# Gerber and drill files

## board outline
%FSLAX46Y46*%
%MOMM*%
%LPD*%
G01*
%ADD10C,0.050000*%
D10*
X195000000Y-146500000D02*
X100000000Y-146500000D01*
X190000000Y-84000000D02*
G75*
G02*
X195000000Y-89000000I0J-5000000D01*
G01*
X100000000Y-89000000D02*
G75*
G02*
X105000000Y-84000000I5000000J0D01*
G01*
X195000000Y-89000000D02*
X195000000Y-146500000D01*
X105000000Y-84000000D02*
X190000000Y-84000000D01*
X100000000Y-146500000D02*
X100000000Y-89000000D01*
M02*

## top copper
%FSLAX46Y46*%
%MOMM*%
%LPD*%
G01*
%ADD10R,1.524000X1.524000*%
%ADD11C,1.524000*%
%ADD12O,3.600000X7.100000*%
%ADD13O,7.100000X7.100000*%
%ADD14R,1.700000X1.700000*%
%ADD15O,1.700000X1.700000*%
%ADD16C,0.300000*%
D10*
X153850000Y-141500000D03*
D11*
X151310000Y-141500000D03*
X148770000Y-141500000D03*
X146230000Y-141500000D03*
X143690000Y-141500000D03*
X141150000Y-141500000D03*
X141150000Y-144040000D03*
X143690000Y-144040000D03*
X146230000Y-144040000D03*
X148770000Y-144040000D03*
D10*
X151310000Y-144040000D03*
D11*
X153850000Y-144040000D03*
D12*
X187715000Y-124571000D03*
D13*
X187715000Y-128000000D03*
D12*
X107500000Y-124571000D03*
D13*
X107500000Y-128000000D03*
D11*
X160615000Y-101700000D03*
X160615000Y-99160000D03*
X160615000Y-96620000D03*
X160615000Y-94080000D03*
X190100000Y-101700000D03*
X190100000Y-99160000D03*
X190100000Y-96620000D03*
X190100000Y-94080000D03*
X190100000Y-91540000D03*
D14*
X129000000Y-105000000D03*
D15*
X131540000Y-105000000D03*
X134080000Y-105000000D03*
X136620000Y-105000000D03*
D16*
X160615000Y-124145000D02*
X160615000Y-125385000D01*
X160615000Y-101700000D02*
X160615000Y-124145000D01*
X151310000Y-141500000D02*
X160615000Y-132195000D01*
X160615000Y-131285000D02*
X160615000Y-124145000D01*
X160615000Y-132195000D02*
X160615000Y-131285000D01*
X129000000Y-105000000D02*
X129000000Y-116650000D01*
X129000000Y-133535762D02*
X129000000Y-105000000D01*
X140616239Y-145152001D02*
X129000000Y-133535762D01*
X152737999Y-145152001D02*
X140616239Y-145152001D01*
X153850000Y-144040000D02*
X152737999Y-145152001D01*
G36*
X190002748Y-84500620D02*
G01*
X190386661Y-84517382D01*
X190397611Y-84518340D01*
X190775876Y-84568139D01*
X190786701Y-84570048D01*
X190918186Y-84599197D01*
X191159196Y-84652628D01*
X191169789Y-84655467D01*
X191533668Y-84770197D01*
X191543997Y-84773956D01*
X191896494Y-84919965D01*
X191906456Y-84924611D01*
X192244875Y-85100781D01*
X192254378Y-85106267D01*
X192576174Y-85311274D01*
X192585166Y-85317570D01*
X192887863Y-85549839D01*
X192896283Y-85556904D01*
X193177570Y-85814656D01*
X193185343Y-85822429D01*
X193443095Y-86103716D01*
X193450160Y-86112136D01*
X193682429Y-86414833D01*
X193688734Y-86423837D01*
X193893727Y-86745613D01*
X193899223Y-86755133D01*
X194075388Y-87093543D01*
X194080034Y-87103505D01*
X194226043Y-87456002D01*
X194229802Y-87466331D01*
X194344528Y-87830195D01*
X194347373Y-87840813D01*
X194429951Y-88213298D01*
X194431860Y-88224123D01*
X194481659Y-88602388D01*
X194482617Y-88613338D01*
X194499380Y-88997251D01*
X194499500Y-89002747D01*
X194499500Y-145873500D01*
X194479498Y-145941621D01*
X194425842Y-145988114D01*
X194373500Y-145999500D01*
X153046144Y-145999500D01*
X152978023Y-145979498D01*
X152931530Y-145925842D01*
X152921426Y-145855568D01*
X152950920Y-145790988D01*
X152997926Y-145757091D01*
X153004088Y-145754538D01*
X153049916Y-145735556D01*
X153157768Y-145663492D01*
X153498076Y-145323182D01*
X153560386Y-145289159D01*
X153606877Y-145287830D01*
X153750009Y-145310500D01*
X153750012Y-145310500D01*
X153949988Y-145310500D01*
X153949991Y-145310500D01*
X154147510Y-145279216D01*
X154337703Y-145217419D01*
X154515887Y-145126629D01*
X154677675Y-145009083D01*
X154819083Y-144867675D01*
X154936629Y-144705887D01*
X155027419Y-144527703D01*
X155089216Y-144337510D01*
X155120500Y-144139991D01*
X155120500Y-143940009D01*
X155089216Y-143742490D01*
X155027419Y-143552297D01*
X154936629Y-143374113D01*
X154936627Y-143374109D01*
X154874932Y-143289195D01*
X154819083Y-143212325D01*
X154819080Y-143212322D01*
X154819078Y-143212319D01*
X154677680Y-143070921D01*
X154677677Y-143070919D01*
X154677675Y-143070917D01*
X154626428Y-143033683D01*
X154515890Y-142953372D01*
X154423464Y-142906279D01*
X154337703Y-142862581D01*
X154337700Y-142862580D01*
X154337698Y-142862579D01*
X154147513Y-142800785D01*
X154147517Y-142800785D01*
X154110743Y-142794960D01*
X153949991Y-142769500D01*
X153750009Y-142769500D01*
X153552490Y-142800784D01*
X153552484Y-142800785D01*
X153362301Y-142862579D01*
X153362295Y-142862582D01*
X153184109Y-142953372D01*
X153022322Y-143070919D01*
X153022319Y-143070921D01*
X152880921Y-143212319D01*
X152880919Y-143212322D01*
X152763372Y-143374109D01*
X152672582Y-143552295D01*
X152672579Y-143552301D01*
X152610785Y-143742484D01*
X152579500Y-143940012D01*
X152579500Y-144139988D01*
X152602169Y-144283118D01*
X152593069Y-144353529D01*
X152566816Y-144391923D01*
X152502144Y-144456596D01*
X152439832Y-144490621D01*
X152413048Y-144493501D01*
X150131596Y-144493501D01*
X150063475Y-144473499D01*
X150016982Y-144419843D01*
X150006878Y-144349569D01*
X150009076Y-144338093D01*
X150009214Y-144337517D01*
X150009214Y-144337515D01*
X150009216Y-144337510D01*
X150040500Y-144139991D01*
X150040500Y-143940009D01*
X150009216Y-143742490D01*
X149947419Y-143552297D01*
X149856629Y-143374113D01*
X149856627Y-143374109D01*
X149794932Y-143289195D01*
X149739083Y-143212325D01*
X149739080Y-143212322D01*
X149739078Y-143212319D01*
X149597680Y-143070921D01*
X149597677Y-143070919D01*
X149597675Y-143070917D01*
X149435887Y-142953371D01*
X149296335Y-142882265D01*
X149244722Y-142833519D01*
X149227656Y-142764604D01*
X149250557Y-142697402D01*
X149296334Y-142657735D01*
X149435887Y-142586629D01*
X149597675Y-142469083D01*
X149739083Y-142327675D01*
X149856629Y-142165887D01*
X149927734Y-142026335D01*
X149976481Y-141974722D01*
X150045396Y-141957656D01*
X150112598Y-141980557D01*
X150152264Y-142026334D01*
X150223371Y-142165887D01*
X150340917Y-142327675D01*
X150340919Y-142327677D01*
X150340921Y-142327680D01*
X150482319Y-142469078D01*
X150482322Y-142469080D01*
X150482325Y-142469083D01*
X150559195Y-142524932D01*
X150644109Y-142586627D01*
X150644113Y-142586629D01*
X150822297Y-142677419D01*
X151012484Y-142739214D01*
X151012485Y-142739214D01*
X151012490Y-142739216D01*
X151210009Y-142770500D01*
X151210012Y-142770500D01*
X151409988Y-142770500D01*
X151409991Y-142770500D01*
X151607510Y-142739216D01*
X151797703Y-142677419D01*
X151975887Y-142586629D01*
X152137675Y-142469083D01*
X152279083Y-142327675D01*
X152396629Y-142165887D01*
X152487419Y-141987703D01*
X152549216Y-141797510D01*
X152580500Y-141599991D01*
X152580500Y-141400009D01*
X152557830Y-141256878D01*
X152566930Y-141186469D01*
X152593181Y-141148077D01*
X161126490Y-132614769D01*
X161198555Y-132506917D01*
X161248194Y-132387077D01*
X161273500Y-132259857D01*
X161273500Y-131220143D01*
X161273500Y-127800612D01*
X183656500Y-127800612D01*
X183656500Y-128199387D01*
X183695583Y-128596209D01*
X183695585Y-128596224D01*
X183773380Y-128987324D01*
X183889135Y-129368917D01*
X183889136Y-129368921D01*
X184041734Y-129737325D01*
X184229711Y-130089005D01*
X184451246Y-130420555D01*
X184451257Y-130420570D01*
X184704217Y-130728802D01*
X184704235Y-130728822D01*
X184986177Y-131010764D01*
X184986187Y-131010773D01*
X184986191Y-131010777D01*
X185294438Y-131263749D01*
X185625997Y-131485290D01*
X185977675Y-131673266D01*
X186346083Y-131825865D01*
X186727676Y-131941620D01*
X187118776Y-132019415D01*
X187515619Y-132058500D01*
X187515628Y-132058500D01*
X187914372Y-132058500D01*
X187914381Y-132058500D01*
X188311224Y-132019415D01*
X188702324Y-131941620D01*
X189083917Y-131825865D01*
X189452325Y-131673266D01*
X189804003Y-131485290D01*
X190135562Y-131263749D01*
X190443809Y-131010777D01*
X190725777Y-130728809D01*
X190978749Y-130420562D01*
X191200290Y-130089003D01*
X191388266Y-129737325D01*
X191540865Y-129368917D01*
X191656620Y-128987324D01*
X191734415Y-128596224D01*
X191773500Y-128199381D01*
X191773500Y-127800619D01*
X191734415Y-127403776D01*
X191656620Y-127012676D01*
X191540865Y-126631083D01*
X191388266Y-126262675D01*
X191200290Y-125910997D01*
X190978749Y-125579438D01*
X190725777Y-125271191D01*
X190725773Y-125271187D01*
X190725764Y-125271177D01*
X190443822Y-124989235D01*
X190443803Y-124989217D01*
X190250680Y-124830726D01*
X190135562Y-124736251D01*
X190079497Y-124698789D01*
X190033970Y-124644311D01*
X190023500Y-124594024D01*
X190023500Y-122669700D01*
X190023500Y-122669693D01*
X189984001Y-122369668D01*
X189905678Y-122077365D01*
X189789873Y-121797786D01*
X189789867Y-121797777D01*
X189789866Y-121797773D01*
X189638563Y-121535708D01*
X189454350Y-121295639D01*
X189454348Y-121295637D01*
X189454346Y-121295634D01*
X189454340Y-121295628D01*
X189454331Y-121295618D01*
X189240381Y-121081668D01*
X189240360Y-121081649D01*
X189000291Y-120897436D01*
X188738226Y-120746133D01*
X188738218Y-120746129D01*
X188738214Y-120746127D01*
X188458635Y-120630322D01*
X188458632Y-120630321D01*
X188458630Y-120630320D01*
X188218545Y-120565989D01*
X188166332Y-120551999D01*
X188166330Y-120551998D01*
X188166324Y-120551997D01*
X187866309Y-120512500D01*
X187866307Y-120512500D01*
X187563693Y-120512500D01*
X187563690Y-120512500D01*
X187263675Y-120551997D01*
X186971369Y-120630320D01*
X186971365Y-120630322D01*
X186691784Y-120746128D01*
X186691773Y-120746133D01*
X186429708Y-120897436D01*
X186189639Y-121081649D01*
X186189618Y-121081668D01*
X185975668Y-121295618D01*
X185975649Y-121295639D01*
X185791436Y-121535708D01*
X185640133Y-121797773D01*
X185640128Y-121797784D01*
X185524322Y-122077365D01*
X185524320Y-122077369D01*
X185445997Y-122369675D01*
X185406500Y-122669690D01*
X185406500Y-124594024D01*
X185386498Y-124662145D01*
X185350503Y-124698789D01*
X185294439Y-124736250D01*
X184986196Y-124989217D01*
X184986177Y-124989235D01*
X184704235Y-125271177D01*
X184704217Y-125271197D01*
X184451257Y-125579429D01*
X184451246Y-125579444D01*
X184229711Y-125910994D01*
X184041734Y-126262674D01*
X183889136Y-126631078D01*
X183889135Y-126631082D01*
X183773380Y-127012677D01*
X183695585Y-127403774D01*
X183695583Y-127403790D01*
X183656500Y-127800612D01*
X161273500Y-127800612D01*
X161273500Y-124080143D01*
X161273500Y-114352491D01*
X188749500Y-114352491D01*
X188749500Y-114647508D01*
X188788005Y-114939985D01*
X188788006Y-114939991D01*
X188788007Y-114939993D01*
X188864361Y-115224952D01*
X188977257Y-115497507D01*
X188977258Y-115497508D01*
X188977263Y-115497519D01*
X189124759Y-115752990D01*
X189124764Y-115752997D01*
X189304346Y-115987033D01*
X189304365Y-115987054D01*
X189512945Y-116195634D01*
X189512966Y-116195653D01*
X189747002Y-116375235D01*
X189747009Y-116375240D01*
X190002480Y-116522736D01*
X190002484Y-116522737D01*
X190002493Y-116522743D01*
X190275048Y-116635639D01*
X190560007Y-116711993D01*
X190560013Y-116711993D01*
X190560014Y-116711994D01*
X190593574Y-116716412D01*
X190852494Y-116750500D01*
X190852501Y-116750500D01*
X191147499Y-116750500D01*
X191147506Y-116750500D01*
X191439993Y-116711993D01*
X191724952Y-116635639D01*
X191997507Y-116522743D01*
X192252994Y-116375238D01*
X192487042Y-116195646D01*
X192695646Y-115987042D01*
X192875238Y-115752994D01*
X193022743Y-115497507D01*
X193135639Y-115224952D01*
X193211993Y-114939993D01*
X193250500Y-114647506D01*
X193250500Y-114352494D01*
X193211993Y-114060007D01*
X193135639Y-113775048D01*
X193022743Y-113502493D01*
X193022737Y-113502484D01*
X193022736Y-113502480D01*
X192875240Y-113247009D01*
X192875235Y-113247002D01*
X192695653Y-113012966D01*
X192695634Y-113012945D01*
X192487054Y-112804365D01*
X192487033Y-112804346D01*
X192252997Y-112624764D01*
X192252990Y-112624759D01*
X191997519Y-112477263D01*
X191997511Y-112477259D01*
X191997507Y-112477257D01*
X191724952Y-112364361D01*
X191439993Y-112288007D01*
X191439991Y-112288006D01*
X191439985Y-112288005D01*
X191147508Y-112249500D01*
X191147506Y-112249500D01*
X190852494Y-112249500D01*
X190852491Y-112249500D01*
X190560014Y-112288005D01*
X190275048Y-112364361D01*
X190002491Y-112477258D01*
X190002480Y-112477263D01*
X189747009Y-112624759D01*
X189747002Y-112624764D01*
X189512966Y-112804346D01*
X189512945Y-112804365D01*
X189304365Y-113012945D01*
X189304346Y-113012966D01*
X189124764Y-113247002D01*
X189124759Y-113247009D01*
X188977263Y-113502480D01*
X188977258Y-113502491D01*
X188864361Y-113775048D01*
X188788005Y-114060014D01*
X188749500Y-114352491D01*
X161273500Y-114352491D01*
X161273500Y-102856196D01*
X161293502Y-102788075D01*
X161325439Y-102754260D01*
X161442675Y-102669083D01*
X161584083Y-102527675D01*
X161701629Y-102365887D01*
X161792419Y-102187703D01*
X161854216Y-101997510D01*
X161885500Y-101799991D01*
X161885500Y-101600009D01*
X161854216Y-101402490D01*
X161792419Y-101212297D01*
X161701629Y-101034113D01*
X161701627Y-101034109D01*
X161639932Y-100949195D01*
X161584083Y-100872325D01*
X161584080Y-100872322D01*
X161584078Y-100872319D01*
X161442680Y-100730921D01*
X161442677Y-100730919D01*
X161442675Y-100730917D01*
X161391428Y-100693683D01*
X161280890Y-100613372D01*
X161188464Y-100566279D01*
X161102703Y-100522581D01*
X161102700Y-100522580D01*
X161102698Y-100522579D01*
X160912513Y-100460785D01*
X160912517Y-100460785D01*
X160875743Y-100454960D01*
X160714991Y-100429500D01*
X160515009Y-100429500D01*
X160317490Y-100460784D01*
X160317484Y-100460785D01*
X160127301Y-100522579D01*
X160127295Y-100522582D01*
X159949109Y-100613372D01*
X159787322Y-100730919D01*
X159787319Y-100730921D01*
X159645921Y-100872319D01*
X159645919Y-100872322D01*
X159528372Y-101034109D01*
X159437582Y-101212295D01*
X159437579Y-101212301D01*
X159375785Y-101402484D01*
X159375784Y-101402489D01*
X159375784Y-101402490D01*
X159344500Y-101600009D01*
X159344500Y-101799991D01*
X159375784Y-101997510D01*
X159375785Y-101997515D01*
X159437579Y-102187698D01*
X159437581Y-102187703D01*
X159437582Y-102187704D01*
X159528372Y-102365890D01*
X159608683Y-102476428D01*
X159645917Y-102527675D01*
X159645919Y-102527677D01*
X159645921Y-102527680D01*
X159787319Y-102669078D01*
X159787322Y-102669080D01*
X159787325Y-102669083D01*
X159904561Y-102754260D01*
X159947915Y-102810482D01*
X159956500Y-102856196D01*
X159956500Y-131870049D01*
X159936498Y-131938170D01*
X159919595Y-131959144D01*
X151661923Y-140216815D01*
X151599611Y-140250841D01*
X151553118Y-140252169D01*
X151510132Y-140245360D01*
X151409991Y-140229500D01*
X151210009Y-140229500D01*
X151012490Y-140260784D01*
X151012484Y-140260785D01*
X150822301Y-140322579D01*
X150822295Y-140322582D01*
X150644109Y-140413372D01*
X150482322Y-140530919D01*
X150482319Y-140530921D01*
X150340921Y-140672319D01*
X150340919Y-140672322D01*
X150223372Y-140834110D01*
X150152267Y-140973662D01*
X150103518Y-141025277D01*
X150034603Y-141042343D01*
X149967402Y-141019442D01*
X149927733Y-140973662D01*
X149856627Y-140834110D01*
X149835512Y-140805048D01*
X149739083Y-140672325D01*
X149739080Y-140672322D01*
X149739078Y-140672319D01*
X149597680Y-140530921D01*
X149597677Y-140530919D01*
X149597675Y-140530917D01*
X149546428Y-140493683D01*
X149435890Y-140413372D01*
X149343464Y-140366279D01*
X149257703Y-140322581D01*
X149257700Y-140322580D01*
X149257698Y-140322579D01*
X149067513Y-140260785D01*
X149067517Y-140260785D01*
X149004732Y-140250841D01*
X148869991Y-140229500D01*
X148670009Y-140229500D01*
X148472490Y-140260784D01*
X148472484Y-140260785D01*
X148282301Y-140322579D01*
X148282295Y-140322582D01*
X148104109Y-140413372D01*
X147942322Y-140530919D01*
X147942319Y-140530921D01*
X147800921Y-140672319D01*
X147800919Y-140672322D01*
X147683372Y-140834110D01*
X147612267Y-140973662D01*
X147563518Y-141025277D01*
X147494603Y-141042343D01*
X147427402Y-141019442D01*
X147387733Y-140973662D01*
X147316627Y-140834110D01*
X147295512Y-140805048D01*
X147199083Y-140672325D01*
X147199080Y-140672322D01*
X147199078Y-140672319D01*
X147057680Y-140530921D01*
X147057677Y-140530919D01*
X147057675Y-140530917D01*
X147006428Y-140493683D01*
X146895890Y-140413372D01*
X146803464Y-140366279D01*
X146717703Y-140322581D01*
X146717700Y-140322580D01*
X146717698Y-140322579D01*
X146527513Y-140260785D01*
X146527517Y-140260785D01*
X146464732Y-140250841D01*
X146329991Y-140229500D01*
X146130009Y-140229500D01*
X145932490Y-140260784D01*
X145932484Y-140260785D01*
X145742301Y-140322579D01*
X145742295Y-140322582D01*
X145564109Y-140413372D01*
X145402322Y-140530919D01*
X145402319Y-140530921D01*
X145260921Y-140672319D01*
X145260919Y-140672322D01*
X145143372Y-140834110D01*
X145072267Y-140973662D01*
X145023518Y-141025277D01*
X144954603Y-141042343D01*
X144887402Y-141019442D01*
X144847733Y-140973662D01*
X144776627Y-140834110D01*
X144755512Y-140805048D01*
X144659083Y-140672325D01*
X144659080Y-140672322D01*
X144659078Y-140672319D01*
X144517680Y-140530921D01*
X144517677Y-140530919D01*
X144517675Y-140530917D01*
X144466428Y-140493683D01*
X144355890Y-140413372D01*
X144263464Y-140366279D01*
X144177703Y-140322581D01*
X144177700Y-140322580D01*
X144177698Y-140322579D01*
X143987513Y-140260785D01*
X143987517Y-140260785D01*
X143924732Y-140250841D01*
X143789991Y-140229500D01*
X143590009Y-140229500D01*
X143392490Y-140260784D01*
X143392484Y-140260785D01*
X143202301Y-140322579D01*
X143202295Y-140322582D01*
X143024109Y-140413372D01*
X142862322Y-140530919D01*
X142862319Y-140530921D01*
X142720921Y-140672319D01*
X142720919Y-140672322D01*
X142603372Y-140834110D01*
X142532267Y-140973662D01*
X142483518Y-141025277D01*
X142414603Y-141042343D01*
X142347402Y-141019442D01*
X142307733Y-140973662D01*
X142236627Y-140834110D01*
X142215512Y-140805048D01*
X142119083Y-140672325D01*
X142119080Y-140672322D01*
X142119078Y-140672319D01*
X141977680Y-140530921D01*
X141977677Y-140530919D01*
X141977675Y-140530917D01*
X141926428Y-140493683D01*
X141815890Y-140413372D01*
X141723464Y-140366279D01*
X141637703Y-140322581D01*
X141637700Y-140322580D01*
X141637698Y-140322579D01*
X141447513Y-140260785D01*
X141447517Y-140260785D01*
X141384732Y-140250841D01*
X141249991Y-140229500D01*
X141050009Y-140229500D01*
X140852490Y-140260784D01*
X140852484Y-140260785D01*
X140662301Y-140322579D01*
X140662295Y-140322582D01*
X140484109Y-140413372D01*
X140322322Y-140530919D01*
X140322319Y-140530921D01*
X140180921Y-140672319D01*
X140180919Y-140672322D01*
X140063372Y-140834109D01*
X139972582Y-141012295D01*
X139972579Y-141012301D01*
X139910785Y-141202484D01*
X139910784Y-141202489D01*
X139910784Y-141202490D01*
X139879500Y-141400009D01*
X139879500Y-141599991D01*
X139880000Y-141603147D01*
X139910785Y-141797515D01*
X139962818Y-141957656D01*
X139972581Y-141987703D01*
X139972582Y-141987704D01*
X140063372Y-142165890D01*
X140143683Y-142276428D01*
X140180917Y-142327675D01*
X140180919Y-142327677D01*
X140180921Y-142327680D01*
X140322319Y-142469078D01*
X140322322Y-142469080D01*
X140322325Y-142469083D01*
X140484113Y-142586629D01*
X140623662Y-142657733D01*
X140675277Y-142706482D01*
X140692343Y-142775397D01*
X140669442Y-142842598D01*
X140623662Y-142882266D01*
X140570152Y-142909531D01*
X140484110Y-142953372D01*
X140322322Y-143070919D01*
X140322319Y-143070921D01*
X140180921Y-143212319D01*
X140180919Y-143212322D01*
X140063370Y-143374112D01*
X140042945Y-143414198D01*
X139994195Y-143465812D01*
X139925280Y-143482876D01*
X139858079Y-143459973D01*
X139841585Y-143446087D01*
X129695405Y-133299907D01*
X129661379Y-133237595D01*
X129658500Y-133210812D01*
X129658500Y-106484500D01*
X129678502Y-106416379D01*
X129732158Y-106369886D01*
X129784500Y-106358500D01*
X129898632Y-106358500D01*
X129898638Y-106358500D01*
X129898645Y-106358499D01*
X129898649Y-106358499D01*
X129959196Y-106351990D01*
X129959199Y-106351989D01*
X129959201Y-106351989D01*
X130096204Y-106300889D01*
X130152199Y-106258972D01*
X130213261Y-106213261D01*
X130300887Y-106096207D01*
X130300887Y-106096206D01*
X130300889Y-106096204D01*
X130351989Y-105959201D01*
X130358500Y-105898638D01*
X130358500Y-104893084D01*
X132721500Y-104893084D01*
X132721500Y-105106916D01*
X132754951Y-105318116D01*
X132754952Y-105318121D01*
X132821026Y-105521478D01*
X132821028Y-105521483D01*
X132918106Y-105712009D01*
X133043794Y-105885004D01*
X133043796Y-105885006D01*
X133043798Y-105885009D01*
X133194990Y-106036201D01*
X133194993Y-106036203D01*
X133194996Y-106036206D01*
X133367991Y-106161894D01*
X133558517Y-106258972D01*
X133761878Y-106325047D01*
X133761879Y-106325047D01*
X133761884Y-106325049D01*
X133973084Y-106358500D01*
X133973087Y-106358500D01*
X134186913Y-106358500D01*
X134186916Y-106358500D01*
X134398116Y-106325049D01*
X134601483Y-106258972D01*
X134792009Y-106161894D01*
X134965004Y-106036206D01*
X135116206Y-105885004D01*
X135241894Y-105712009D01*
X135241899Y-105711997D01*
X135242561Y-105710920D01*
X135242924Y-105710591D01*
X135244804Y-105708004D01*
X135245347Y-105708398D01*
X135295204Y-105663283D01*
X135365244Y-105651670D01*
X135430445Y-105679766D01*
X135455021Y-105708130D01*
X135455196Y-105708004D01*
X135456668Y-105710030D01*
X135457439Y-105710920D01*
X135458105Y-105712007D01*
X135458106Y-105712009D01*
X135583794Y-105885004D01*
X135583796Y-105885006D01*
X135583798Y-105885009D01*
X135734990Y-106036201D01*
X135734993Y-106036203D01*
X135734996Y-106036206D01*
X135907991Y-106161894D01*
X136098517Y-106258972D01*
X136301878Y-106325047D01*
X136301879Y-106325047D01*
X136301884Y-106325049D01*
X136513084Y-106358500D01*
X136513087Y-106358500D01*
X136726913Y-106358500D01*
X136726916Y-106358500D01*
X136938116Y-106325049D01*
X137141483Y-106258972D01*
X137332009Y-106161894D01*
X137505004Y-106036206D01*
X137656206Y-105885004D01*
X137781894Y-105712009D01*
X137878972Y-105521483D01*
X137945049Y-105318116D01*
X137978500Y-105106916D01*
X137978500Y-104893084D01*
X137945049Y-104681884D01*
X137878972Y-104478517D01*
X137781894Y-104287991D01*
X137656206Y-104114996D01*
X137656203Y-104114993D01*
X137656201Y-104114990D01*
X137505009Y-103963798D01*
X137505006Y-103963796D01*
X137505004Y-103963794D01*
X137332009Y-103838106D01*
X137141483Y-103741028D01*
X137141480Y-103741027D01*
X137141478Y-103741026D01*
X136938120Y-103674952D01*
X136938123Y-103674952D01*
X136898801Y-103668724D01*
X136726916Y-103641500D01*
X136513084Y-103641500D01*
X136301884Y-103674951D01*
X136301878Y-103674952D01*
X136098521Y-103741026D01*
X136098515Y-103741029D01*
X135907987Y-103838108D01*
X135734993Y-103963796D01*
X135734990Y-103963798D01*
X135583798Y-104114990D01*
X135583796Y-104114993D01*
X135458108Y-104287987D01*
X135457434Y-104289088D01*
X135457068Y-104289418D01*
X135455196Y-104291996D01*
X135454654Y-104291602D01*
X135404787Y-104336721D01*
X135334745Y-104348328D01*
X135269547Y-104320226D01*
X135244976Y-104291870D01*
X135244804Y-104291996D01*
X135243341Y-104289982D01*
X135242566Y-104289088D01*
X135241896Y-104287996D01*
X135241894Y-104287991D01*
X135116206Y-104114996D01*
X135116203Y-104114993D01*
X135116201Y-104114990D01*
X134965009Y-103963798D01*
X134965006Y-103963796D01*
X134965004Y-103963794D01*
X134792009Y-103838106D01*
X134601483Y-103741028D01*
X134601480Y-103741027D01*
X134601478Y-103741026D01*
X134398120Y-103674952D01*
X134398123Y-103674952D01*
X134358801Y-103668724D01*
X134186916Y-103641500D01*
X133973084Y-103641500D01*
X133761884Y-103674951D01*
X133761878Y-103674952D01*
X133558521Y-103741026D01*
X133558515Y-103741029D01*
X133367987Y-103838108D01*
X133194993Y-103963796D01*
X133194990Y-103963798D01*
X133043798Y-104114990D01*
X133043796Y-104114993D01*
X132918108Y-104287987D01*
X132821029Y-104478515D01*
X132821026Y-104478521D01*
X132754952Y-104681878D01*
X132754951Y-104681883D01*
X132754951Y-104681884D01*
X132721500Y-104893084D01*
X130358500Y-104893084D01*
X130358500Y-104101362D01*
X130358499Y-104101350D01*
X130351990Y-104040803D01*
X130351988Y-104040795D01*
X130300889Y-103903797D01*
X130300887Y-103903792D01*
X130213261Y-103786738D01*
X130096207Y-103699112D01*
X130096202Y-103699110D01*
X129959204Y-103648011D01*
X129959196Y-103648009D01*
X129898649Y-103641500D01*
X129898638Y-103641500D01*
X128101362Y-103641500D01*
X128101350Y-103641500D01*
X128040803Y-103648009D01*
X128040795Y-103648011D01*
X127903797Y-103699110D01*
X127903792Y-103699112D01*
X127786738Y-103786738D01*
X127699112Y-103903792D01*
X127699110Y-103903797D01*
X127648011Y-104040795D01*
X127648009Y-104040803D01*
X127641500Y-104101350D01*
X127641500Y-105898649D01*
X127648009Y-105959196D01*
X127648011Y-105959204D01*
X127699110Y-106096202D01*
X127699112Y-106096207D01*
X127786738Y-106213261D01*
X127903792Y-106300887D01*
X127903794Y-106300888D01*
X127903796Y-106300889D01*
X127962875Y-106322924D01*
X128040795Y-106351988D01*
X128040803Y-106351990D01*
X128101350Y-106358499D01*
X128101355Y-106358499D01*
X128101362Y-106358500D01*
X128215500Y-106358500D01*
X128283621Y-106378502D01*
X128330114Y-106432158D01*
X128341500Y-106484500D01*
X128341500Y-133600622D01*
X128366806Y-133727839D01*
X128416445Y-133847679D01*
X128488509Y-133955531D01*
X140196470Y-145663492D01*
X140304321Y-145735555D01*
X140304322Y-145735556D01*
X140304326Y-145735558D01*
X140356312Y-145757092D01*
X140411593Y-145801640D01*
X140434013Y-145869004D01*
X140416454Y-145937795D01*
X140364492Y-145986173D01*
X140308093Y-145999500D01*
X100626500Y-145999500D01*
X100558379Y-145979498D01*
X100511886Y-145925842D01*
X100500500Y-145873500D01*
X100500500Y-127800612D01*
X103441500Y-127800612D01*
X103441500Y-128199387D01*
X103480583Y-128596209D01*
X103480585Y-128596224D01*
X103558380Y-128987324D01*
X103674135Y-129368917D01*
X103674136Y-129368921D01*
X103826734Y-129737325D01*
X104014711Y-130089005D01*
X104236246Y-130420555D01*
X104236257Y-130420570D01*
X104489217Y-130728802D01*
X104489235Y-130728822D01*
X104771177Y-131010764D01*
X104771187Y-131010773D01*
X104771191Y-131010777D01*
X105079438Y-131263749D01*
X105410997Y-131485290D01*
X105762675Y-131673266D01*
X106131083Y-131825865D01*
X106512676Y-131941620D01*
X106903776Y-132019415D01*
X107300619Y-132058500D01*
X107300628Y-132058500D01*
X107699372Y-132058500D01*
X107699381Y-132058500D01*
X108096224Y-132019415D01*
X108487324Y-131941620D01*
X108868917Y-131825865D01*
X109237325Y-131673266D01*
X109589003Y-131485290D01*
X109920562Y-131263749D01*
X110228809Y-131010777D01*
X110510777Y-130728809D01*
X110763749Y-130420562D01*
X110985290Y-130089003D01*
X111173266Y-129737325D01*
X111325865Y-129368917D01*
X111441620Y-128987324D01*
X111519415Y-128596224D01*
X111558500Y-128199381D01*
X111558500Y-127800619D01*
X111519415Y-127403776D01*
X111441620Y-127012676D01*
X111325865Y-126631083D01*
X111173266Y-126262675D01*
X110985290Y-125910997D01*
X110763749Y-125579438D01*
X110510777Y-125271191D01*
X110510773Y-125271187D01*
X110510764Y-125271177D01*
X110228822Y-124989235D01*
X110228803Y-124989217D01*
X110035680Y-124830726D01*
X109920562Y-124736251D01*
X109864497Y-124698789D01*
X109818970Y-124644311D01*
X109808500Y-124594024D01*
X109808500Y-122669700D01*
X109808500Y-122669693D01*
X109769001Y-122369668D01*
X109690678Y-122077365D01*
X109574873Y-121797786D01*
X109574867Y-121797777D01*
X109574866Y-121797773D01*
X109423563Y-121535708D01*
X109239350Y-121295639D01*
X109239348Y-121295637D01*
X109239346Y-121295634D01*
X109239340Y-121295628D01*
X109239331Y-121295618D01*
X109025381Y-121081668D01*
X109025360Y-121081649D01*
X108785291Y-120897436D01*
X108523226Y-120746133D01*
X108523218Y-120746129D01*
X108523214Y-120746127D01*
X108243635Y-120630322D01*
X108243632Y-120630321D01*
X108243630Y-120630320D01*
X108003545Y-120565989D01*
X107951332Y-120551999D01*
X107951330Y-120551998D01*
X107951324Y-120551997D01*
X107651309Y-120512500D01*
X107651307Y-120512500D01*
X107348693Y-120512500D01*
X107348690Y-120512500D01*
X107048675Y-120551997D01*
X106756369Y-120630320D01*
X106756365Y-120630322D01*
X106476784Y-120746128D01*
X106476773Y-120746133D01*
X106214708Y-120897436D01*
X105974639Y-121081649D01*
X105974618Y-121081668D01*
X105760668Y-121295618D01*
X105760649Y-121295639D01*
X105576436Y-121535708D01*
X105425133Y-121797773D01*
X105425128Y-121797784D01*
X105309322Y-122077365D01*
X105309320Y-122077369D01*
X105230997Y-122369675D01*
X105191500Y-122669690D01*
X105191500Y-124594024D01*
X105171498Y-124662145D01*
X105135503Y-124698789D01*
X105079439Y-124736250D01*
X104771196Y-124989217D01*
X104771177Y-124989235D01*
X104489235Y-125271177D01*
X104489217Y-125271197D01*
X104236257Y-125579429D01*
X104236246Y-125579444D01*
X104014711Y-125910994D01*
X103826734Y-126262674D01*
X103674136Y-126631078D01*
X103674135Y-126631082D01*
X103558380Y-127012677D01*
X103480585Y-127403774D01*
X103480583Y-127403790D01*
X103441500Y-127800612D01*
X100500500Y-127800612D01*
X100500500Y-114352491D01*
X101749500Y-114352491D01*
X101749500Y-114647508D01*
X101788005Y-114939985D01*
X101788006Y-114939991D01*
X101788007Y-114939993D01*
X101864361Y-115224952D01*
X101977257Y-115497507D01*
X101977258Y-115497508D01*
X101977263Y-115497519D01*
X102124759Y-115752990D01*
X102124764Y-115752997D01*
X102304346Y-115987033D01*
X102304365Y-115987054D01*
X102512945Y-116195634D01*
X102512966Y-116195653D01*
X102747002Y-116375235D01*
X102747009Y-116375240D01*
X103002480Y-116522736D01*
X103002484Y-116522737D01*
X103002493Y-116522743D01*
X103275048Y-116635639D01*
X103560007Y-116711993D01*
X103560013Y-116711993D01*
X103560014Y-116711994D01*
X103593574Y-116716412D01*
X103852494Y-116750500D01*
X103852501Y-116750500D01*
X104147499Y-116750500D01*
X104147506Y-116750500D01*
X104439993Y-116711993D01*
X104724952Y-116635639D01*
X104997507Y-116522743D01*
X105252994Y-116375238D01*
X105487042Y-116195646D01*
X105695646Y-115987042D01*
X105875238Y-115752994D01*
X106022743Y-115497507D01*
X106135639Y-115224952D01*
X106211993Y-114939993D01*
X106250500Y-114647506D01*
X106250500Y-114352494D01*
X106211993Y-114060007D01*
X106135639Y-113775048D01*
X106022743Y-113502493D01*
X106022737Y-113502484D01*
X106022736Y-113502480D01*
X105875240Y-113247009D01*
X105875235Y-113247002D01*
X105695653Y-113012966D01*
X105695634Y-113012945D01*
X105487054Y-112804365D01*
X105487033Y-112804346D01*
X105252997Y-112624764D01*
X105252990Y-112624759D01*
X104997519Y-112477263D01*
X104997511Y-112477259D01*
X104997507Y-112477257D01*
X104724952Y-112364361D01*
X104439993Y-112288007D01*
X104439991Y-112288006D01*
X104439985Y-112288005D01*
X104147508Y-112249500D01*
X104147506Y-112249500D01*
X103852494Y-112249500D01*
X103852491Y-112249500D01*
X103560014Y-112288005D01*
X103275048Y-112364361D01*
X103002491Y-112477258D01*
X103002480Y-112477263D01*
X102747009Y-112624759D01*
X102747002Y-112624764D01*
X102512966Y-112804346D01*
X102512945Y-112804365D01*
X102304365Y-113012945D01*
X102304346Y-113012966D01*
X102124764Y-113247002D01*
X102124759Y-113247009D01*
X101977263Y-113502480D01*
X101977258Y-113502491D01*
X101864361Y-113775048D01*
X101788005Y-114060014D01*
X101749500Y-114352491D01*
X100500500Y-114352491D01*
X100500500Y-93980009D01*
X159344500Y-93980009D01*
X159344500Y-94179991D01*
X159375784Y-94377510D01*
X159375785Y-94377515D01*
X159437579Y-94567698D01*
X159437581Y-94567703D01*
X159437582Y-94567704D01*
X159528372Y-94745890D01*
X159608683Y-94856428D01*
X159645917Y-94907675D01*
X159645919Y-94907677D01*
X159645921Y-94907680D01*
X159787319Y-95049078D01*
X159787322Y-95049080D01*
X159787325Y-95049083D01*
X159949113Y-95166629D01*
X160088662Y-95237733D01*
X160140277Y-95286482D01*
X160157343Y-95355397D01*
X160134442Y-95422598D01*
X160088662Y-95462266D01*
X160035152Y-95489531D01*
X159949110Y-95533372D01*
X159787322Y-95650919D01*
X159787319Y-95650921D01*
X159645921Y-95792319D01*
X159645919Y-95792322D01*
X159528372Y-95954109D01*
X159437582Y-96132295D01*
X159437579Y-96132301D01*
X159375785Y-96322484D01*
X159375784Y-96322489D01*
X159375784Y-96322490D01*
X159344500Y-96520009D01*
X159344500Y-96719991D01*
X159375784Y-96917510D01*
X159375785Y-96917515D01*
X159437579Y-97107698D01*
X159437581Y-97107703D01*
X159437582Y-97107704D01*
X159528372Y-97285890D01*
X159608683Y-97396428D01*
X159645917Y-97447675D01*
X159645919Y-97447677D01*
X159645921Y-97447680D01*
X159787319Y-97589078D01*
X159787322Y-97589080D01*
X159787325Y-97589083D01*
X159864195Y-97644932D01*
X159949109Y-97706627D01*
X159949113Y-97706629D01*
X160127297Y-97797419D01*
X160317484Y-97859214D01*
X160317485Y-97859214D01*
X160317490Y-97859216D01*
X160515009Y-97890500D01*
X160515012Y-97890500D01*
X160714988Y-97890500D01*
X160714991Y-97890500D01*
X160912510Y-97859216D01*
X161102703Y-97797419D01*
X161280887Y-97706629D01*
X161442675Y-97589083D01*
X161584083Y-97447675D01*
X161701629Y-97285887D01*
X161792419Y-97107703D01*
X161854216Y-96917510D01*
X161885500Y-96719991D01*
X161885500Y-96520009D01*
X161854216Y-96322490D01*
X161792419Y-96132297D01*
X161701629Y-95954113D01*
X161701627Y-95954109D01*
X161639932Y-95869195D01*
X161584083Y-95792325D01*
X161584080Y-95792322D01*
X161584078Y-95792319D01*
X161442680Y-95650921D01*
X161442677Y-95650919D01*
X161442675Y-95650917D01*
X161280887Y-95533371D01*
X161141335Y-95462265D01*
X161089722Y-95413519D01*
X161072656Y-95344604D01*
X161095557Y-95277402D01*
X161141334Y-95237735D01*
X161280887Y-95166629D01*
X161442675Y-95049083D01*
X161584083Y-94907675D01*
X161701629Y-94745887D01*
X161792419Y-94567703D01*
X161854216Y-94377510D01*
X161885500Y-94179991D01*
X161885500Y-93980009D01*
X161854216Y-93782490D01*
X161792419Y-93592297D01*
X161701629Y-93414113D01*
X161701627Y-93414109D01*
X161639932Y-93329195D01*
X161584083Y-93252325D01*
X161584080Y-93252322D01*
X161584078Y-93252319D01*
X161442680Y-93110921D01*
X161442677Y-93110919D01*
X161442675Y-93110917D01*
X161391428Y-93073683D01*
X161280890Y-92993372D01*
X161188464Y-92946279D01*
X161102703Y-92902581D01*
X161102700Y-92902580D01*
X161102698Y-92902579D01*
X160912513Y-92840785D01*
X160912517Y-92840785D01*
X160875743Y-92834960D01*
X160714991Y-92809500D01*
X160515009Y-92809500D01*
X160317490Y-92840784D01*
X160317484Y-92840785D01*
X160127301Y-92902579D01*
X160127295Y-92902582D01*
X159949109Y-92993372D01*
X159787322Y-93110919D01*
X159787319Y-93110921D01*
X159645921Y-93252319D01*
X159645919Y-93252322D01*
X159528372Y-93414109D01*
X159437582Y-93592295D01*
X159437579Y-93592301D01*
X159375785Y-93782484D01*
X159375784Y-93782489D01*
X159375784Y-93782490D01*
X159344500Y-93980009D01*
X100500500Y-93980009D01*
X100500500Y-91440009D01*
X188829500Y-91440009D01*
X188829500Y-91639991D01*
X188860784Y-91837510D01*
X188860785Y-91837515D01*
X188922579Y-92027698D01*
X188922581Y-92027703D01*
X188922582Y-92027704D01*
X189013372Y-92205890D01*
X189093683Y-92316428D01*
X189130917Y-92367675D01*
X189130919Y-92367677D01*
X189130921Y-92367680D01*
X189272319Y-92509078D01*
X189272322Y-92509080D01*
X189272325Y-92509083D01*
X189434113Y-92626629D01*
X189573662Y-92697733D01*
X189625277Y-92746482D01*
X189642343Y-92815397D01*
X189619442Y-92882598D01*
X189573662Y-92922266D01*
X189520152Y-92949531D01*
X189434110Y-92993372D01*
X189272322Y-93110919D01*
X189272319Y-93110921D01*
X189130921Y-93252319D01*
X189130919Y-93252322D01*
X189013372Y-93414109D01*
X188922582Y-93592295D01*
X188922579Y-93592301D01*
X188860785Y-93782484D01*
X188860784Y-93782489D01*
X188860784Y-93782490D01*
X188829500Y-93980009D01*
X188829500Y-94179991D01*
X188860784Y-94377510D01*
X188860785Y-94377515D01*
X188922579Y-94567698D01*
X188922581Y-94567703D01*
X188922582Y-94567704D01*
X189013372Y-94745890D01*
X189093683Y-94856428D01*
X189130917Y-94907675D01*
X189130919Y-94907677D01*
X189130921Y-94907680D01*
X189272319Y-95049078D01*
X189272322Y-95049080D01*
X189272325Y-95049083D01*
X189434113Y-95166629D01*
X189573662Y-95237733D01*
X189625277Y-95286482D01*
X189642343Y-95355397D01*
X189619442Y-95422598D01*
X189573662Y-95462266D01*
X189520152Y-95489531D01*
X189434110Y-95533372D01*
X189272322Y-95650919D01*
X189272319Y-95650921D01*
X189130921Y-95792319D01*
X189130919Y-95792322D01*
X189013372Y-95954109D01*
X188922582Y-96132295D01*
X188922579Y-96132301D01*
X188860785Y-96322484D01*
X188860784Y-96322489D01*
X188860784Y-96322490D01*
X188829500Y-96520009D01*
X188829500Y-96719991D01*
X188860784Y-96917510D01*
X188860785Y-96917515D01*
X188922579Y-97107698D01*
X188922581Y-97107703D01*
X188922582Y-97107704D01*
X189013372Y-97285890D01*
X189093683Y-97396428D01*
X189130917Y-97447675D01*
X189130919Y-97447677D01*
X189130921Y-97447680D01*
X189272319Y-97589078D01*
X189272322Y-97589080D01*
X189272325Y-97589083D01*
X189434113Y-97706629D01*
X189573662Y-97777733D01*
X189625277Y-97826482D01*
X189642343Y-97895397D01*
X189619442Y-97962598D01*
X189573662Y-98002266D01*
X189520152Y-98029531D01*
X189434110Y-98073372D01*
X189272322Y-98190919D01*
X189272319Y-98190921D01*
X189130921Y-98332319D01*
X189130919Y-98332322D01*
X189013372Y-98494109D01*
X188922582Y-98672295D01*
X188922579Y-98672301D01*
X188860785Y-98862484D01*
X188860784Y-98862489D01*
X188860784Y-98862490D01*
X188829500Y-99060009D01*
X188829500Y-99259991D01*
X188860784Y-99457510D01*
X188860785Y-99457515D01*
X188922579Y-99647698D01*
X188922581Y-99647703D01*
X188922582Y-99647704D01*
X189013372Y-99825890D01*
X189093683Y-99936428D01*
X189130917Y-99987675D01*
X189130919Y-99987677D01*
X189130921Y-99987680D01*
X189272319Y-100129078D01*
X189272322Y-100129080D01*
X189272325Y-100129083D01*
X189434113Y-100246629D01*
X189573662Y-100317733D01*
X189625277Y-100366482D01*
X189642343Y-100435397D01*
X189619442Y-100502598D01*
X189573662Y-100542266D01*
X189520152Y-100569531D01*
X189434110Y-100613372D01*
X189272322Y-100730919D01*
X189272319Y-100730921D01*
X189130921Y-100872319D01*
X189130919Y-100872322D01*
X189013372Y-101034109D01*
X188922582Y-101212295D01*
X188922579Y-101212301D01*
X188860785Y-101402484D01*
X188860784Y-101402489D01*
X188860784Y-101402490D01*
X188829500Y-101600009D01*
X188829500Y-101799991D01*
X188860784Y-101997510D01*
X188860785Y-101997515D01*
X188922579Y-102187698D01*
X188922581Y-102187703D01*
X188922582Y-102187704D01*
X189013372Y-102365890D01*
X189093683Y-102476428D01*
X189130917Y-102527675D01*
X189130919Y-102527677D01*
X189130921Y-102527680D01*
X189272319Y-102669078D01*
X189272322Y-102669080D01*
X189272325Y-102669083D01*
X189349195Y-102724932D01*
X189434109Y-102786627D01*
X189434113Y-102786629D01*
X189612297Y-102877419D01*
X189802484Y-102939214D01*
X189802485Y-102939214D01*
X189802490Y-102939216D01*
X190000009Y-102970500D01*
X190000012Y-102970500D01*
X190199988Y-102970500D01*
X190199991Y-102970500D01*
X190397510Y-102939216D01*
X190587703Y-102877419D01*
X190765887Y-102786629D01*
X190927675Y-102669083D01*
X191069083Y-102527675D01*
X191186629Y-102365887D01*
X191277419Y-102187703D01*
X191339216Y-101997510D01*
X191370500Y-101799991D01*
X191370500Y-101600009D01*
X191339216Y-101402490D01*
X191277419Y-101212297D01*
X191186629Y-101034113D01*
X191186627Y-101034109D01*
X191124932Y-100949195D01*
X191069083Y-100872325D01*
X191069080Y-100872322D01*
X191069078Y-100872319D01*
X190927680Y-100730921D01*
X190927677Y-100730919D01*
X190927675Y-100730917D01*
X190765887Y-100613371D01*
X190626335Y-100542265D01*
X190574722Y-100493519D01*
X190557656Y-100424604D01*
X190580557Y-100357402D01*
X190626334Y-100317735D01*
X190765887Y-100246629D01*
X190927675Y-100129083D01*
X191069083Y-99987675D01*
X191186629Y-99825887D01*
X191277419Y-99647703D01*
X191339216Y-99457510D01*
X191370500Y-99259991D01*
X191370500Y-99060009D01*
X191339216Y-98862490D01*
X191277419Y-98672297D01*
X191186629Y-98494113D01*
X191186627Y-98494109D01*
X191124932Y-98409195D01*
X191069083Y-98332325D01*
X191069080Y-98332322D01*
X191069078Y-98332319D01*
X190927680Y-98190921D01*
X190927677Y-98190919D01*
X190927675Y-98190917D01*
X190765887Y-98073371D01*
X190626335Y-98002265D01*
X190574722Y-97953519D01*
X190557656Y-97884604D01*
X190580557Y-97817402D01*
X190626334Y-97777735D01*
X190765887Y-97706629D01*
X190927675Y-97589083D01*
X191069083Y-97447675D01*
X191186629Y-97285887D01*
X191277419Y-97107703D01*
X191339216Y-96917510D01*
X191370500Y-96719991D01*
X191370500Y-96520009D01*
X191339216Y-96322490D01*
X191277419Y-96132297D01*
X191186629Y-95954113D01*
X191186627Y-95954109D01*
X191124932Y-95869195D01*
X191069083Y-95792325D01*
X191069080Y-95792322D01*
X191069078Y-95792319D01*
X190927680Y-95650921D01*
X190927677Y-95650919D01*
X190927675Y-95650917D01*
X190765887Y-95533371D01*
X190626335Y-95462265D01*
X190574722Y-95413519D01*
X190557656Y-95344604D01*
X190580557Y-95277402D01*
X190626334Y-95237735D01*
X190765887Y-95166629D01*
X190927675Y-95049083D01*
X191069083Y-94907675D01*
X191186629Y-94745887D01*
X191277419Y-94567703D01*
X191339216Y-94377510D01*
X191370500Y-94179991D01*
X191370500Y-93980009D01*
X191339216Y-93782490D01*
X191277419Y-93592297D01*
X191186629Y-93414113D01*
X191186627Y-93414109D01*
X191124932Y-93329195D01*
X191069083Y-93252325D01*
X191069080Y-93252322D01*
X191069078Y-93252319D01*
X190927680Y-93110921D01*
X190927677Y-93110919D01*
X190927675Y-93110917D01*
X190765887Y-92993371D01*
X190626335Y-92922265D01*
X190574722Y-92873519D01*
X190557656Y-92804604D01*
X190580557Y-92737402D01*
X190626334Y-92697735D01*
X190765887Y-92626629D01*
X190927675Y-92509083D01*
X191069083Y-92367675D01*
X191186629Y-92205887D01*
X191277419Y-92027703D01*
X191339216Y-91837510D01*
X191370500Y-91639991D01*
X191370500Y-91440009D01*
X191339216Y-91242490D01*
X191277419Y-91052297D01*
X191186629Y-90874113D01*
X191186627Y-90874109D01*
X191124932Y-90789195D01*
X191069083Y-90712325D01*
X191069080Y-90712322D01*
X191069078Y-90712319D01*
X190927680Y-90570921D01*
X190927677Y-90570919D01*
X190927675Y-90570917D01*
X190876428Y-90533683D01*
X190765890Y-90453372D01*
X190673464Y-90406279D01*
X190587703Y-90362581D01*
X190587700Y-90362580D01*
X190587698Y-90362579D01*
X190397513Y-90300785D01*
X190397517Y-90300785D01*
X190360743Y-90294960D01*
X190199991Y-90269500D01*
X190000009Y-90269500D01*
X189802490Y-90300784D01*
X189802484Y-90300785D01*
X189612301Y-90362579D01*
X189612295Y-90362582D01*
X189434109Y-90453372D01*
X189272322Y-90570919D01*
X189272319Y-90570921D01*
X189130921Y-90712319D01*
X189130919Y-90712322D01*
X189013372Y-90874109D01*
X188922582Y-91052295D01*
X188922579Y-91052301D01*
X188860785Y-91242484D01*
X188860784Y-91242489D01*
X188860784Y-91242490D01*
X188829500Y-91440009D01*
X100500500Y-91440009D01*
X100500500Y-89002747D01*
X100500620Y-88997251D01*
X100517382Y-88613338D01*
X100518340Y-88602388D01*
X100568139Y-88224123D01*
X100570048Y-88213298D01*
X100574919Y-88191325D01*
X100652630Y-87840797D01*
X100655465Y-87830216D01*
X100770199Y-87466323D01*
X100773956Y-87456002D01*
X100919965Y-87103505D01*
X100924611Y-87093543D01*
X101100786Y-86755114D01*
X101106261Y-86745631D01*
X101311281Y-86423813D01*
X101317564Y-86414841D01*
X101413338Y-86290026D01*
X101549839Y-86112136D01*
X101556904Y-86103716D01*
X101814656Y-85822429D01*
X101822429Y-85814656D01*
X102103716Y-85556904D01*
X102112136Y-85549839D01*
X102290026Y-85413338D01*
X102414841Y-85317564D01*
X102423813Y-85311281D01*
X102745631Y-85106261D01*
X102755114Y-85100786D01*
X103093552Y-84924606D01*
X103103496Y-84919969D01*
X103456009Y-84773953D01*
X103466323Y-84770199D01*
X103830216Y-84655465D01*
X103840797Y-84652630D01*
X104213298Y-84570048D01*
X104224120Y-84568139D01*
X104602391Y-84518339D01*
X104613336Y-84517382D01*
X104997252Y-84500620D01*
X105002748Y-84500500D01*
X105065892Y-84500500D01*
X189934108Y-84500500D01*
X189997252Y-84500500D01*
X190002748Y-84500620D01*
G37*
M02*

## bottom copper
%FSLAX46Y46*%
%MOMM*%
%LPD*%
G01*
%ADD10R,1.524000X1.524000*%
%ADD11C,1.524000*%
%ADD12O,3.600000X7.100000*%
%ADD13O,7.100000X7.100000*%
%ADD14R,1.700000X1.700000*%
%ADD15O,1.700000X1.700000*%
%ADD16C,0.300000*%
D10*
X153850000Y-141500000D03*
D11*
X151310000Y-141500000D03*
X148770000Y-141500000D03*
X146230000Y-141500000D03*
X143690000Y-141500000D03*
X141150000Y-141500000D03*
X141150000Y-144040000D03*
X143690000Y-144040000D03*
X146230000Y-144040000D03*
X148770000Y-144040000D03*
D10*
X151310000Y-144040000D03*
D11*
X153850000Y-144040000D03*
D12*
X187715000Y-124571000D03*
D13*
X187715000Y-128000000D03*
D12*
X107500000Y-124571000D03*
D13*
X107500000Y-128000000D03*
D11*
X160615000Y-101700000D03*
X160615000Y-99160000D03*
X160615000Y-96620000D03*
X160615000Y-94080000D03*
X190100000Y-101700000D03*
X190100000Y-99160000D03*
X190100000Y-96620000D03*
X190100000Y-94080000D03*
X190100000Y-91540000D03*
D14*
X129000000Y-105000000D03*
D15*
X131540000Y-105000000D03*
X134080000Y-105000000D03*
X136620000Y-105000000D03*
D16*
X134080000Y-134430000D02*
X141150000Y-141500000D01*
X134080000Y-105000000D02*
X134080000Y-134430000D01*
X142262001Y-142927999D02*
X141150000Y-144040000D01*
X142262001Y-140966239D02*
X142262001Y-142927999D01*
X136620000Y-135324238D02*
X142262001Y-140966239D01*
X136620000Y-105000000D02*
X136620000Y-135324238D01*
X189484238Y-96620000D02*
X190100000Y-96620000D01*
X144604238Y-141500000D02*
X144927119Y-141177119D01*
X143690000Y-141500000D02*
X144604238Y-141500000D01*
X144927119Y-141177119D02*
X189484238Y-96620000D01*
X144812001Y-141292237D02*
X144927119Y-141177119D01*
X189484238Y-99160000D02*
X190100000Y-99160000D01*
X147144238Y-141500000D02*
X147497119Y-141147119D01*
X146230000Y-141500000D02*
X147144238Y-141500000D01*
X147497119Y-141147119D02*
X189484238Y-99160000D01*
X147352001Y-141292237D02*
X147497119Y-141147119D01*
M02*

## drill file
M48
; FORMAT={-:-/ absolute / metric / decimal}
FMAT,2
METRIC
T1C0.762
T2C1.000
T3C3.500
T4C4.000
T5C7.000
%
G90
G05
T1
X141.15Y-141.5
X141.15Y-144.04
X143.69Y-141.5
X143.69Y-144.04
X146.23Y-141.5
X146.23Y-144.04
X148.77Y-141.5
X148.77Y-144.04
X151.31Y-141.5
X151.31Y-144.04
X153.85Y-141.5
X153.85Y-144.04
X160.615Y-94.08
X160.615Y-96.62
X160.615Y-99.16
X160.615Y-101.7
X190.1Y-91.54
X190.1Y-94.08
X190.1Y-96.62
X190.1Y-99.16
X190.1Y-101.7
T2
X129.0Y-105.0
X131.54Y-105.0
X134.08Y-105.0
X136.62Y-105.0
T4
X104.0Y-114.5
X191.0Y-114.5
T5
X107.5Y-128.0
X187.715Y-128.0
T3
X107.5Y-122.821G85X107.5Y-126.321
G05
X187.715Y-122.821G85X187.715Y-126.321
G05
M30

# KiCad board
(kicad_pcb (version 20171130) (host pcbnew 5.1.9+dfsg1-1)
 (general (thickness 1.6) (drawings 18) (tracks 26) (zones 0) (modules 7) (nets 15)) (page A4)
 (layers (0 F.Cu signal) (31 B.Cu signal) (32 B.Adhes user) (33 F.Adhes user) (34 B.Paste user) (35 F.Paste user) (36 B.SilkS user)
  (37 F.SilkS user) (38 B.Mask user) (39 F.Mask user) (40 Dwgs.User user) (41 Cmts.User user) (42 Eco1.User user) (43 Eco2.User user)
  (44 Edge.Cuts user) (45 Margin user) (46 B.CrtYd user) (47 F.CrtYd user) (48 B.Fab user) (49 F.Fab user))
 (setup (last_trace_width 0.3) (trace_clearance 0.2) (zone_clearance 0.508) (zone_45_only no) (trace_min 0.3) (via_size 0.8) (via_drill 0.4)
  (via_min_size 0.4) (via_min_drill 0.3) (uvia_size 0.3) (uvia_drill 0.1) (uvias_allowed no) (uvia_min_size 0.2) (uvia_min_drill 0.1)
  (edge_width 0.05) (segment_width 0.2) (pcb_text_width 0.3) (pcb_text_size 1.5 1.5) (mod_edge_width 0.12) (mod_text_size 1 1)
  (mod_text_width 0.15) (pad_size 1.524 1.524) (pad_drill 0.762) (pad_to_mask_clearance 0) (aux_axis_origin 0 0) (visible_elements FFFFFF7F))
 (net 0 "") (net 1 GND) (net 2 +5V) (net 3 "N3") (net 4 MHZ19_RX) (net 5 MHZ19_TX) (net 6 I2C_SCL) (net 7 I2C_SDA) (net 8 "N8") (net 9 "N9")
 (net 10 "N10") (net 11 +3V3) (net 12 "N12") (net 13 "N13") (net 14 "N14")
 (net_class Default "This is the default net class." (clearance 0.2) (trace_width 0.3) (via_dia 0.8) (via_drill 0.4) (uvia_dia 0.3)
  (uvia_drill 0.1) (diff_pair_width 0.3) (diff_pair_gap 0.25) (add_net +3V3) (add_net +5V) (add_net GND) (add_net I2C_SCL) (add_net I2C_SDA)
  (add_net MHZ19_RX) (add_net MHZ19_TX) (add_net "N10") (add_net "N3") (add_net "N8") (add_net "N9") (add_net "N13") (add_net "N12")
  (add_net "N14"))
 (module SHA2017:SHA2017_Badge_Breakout (layer F.Cu) (at 147.5 137.944)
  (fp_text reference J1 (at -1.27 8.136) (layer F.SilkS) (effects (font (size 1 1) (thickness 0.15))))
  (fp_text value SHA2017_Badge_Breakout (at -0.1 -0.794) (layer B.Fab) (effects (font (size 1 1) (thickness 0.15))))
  (pad 1 thru_hole rect (at 6.35 3.556) (size 1.524 1.524) (drill 0.762) (layers *.Cu *.Mask) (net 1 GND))
  (pad 2 thru_hole circle (at 3.81 3.556) (size 1.524 1.524) (drill 0.762) (layers *.Cu *.Mask) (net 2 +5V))
  (pad 3 thru_hole circle (at 1.27 3.556) (size 1.524 1.524) (drill 0.762) (layers *.Cu *.Mask) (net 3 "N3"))
  (pad 4 thru_hole circle (at -1.27 3.556) (size 1.524 1.524) (drill 0.762) (layers *.Cu *.Mask) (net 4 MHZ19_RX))
  (pad 5 thru_hole circle (at -3.81 3.556) (size 1.524 1.524) (drill 0.762) (layers *.Cu *.Mask) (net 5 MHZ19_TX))
  (pad 6 thru_hole circle (at -6.35 3.556) (size 1.524 1.524) (drill 0.762) (layers *.Cu *.Mask) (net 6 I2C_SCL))
  (pad 7 thru_hole circle (at -6.35 6.096) (size 1.524 1.524) (drill 0.762) (layers *.Cu *.Mask) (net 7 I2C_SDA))
  (pad 8 thru_hole circle (at -3.81 6.096) (size 1.524 1.524) (drill 0.762) (layers *.Cu *.Mask) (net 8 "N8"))
  (pad 9 thru_hole circle (at -1.27 6.096) (size 1.524 1.524) (drill 0.762) (layers *.Cu *.Mask) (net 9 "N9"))
  (pad 10 thru_hole circle (at 1.27 6.096) (size 1.524 1.524) (drill 0.762) (layers *.Cu *.Mask) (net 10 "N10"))
  (pad 11 thru_hole rect (at 3.81 6.096) (size 1.524 1.524) (drill 0.762) (layers *.Cu *.Mask) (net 1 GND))
  (pad 12 thru_hole circle (at 6.35 6.096) (size 1.524 1.524) (drill 0.762) (layers *.Cu *.Mask) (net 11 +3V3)))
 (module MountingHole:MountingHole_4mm (layer F.Cu) (at 191 114.5)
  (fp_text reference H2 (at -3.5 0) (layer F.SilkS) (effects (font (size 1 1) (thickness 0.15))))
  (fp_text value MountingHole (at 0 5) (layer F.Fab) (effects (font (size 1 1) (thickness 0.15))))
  (pad 1 np_thru_hole circle (at 0 0) (size 4 4) (drill 4) (layers *.Cu *.Mask)))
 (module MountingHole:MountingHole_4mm (layer F.Cu) (at 104 114.5)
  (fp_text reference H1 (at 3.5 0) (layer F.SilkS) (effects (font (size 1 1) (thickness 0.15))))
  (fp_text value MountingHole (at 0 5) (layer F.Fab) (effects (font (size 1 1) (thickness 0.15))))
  (pad 1 np_thru_hole circle (at 0 0) (size 4 4) (drill 4) (layers *.Cu *.Mask)))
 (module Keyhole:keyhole (layer F.Cu) (at 182 126.349)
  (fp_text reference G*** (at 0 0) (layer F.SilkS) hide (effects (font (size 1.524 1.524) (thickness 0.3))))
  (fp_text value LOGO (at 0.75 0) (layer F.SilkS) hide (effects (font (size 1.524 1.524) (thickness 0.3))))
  (pad "" np_thru_hole oval (at 5.715 -1.778) (size 3.6 7.1) (drill oval 3.5 7) (layers *.Cu *.Mask))
  (pad "" np_thru_hole oval (at 5.715 1.651) (size 7.1 7.1) (drill oval 7) (layers *.Cu *.Mask)))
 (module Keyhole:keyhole (layer F.Cu) (at 101.785 126.349)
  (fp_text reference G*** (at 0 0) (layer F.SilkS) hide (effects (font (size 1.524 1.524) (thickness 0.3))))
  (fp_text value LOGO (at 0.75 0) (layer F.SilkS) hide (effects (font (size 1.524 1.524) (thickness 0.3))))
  (pad "" np_thru_hole oval (at 5.715 -1.778) (size 3.6 7.1) (drill oval 3.5 7) (layers *.Cu *.Mask))
  (pad "" np_thru_hole oval (at 5.715 1.651) (size 7.1 7.1) (drill oval 7) (layers *.Cu *.Mask)))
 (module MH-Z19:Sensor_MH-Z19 (layer F.Cu) (at 190 89)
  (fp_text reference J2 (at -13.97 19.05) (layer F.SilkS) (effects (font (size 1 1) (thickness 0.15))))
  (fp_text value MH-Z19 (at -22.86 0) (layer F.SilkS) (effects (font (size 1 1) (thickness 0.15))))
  (pad 1 thru_hole circle (at -29.385 12.7) (size 1.524 1.524) (drill 0.762) (layers *.Cu *.Mask) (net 2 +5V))
  (pad 2 thru_hole circle (at -29.385 10.16) (size 1.524 1.524) (drill 0.762) (layers *.Cu *.Mask) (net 1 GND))
  (pad "" thru_hole circle (at -29.385 7.62) (size 1.524 1.524) (drill 0.762) (layers *.Cu *.Mask))
  (pad 4 thru_hole circle (at -29.385 5.08) (size 1.524 1.524) (drill 0.762) (layers *.Cu *.Mask) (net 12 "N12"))
  (pad 3 thru_hole circle (at 0.1 12.7) (size 1.524 1.524) (drill 0.762) (layers *.Cu *.Mask) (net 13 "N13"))
  (pad 6 thru_hole circle (at 0.1 10.16) (size 1.524 1.524) (drill 0.762) (layers *.Cu *.Mask) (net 4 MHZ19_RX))
  (pad 7 thru_hole circle (at 0.1 7.62) (size 1.524 1.524) (drill 0.762) (layers *.Cu *.Mask) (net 5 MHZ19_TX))
  (pad "" thru_hole circle (at 0.1 5.08) (size 1.524 1.524) (drill 0.762) (layers *.Cu *.Mask))
  (pad 5 thru_hole circle (at 0.1 2.54) (size 1.524 1.524) (drill 0.762) (layers *.Cu *.Mask) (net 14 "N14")))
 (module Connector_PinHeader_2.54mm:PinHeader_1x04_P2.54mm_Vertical (layer F.Cu) (at 129 105 90)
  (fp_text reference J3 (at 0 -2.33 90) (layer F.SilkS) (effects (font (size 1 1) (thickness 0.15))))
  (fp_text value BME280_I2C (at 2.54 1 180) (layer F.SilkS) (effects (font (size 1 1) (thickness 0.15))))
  (pad 1 thru_hole rect (at 0 0 90) (size 1.7 1.7) (drill 1) (layers *.Cu *.Mask) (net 11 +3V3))
  (pad 2 thru_hole oval (at 0 2.54 90) (size 1.7 1.7) (drill 1) (layers *.Cu *.Mask) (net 1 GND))
  (pad 3 thru_hole oval (at 0 5.08 90) (size 1.7 1.7) (drill 1) (layers *.Cu *.Mask) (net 6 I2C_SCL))
  (pad 4 thru_hole oval (at 0 7.62 90) (size 1.7 1.7) (drill 1) (layers *.Cu *.Mask) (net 7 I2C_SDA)))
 (gr_line (start 195 146.5) (end 100 146.5) (layer Edge.Cuts) (width 0.05))
 (gr_arc (start 190 89) (end 195 89) (angle -90) (layer Edge.Cuts) (width 0.05))
 (gr_arc (start 105 89) (end 105 84) (angle -90) (layer Edge.Cuts) (width 0.05))
 (gr_line (start 195 89) (end 195 146.5) (layer Edge.Cuts) (width 0.05))
 (gr_line (start 105 84) (end 190 84) (layer Edge.Cuts) (width 0.05))
 (gr_line (start 100 146.5) (end 100 89) (layer Edge.Cuts) (width 0.05))
 (segment (start 160.615 124.145) (end 160.615 125.385) (width 0.3) (layer F.Cu) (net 2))
 (segment (start 160.615 101.7) (end 160.615 124.145) (width 0.3) (layer F.Cu) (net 2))
 (segment (start 151.31 141.5) (end 160.615 132.195) (width 0.3) (layer F.Cu) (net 2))
 (segment (start 160.615 131.285) (end 160.615 124.145) (width 0.3) (layer F.Cu) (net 2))
 (segment (start 160.615 132.195) (end 160.615 131.285) (width 0.3) (layer F.Cu) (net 2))
 (segment (start 134.08 134.43) (end 141.15 141.5) (width 0.3) (layer B.Cu) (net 6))
 (segment (start 134.08 105) (end 134.08 134.43) (width 0.3) (layer B.Cu) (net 6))
 (segment (start 142.262001 142.927999) (end 141.15 144.04) (width 0.3) (layer B.Cu) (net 7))
 (segment (start 142.262001 140.966239) (end 142.262001 142.927999) (width 0.3) (layer B.Cu) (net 7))
 (segment (start 136.62 135.324238) (end 142.262001 140.966239) (width 0.3) (layer B.Cu) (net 7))
 (segment (start 136.62 105) (end 136.62 135.324238) (width 0.3) (layer B.Cu) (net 7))
 (segment (start 129 105) (end 129 116.65) (width 0.3) (layer F.Cu) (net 11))
 (segment (start 129 133.535762) (end 129 105) (width 0.3) (layer F.Cu) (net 11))
 (segment (start 140.616239 145.152001) (end 129 133.535762) (width 0.3) (layer F.Cu) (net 11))
 (segment (start 152.737999 145.152001) (end 140.616239 145.152001) (width 0.3) (layer F.Cu) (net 11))
 (segment (start 153.85 144.04) (end 152.737999 145.152001) (width 0.3) (layer F.Cu) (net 11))
 (segment (start 189.484238 96.62) (end 190.1 96.62) (width 0.3) (layer B.Cu) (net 5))
 (segment (start 144.604238 141.5) (end 144.927119 141.177119) (width 0.3) (layer B.Cu) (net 5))
 (segment (start 143.69 141.5) (end 144.604238 141.5) (width 0.3) (layer B.Cu) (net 5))
 (segment (start 144.927119 141.177119) (end 189.484238 96.62) (width 0.3) (layer B.Cu) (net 5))
 (segment (start 144.812001 141.292237) (end 144.927119 141.177119) (width 0.3) (layer B.Cu) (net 5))
 (segment (start 189.484238 99.16) (end 190.1 99.16) (width 0.3) (layer B.Cu) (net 4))
 (segment (start 147.144238 141.5) (end 147.497119 141.147119) (width 0.3) (layer B.Cu) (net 4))
 (segment (start 146.23 141.5) (end 147.144238 141.5) (width 0.3) (layer B.Cu) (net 4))
 (segment (start 147.497119 141.147119) (end 189.484238 99.16) (width 0.3) (layer B.Cu) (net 4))
 (segment (start 147.352001 141.292237) (end 147.497119 141.147119) (width 0.3) (layer B.Cu) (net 4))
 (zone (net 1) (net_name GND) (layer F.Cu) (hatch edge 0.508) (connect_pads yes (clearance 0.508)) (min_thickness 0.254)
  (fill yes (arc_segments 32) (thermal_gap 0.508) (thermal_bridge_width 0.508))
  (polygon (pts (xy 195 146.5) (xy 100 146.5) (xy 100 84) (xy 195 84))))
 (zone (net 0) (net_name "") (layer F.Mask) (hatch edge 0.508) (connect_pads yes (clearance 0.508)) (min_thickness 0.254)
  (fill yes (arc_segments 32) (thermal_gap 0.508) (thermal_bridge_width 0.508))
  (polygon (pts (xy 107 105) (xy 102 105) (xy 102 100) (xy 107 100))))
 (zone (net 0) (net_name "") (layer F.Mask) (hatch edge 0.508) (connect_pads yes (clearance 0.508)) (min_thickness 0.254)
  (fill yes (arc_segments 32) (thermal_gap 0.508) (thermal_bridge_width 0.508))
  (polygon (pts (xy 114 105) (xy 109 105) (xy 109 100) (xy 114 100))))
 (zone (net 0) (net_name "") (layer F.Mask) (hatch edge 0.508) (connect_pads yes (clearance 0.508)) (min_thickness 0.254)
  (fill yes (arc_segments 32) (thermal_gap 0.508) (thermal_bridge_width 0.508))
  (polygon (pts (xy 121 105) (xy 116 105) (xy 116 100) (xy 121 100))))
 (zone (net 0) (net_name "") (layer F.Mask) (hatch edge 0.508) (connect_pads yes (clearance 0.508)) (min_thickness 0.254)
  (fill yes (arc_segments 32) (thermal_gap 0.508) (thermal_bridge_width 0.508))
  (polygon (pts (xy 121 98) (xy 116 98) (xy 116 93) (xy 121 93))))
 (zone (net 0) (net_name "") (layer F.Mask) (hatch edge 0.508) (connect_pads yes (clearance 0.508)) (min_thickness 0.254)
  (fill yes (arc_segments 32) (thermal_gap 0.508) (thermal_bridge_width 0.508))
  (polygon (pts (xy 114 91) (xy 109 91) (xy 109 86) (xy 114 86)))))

